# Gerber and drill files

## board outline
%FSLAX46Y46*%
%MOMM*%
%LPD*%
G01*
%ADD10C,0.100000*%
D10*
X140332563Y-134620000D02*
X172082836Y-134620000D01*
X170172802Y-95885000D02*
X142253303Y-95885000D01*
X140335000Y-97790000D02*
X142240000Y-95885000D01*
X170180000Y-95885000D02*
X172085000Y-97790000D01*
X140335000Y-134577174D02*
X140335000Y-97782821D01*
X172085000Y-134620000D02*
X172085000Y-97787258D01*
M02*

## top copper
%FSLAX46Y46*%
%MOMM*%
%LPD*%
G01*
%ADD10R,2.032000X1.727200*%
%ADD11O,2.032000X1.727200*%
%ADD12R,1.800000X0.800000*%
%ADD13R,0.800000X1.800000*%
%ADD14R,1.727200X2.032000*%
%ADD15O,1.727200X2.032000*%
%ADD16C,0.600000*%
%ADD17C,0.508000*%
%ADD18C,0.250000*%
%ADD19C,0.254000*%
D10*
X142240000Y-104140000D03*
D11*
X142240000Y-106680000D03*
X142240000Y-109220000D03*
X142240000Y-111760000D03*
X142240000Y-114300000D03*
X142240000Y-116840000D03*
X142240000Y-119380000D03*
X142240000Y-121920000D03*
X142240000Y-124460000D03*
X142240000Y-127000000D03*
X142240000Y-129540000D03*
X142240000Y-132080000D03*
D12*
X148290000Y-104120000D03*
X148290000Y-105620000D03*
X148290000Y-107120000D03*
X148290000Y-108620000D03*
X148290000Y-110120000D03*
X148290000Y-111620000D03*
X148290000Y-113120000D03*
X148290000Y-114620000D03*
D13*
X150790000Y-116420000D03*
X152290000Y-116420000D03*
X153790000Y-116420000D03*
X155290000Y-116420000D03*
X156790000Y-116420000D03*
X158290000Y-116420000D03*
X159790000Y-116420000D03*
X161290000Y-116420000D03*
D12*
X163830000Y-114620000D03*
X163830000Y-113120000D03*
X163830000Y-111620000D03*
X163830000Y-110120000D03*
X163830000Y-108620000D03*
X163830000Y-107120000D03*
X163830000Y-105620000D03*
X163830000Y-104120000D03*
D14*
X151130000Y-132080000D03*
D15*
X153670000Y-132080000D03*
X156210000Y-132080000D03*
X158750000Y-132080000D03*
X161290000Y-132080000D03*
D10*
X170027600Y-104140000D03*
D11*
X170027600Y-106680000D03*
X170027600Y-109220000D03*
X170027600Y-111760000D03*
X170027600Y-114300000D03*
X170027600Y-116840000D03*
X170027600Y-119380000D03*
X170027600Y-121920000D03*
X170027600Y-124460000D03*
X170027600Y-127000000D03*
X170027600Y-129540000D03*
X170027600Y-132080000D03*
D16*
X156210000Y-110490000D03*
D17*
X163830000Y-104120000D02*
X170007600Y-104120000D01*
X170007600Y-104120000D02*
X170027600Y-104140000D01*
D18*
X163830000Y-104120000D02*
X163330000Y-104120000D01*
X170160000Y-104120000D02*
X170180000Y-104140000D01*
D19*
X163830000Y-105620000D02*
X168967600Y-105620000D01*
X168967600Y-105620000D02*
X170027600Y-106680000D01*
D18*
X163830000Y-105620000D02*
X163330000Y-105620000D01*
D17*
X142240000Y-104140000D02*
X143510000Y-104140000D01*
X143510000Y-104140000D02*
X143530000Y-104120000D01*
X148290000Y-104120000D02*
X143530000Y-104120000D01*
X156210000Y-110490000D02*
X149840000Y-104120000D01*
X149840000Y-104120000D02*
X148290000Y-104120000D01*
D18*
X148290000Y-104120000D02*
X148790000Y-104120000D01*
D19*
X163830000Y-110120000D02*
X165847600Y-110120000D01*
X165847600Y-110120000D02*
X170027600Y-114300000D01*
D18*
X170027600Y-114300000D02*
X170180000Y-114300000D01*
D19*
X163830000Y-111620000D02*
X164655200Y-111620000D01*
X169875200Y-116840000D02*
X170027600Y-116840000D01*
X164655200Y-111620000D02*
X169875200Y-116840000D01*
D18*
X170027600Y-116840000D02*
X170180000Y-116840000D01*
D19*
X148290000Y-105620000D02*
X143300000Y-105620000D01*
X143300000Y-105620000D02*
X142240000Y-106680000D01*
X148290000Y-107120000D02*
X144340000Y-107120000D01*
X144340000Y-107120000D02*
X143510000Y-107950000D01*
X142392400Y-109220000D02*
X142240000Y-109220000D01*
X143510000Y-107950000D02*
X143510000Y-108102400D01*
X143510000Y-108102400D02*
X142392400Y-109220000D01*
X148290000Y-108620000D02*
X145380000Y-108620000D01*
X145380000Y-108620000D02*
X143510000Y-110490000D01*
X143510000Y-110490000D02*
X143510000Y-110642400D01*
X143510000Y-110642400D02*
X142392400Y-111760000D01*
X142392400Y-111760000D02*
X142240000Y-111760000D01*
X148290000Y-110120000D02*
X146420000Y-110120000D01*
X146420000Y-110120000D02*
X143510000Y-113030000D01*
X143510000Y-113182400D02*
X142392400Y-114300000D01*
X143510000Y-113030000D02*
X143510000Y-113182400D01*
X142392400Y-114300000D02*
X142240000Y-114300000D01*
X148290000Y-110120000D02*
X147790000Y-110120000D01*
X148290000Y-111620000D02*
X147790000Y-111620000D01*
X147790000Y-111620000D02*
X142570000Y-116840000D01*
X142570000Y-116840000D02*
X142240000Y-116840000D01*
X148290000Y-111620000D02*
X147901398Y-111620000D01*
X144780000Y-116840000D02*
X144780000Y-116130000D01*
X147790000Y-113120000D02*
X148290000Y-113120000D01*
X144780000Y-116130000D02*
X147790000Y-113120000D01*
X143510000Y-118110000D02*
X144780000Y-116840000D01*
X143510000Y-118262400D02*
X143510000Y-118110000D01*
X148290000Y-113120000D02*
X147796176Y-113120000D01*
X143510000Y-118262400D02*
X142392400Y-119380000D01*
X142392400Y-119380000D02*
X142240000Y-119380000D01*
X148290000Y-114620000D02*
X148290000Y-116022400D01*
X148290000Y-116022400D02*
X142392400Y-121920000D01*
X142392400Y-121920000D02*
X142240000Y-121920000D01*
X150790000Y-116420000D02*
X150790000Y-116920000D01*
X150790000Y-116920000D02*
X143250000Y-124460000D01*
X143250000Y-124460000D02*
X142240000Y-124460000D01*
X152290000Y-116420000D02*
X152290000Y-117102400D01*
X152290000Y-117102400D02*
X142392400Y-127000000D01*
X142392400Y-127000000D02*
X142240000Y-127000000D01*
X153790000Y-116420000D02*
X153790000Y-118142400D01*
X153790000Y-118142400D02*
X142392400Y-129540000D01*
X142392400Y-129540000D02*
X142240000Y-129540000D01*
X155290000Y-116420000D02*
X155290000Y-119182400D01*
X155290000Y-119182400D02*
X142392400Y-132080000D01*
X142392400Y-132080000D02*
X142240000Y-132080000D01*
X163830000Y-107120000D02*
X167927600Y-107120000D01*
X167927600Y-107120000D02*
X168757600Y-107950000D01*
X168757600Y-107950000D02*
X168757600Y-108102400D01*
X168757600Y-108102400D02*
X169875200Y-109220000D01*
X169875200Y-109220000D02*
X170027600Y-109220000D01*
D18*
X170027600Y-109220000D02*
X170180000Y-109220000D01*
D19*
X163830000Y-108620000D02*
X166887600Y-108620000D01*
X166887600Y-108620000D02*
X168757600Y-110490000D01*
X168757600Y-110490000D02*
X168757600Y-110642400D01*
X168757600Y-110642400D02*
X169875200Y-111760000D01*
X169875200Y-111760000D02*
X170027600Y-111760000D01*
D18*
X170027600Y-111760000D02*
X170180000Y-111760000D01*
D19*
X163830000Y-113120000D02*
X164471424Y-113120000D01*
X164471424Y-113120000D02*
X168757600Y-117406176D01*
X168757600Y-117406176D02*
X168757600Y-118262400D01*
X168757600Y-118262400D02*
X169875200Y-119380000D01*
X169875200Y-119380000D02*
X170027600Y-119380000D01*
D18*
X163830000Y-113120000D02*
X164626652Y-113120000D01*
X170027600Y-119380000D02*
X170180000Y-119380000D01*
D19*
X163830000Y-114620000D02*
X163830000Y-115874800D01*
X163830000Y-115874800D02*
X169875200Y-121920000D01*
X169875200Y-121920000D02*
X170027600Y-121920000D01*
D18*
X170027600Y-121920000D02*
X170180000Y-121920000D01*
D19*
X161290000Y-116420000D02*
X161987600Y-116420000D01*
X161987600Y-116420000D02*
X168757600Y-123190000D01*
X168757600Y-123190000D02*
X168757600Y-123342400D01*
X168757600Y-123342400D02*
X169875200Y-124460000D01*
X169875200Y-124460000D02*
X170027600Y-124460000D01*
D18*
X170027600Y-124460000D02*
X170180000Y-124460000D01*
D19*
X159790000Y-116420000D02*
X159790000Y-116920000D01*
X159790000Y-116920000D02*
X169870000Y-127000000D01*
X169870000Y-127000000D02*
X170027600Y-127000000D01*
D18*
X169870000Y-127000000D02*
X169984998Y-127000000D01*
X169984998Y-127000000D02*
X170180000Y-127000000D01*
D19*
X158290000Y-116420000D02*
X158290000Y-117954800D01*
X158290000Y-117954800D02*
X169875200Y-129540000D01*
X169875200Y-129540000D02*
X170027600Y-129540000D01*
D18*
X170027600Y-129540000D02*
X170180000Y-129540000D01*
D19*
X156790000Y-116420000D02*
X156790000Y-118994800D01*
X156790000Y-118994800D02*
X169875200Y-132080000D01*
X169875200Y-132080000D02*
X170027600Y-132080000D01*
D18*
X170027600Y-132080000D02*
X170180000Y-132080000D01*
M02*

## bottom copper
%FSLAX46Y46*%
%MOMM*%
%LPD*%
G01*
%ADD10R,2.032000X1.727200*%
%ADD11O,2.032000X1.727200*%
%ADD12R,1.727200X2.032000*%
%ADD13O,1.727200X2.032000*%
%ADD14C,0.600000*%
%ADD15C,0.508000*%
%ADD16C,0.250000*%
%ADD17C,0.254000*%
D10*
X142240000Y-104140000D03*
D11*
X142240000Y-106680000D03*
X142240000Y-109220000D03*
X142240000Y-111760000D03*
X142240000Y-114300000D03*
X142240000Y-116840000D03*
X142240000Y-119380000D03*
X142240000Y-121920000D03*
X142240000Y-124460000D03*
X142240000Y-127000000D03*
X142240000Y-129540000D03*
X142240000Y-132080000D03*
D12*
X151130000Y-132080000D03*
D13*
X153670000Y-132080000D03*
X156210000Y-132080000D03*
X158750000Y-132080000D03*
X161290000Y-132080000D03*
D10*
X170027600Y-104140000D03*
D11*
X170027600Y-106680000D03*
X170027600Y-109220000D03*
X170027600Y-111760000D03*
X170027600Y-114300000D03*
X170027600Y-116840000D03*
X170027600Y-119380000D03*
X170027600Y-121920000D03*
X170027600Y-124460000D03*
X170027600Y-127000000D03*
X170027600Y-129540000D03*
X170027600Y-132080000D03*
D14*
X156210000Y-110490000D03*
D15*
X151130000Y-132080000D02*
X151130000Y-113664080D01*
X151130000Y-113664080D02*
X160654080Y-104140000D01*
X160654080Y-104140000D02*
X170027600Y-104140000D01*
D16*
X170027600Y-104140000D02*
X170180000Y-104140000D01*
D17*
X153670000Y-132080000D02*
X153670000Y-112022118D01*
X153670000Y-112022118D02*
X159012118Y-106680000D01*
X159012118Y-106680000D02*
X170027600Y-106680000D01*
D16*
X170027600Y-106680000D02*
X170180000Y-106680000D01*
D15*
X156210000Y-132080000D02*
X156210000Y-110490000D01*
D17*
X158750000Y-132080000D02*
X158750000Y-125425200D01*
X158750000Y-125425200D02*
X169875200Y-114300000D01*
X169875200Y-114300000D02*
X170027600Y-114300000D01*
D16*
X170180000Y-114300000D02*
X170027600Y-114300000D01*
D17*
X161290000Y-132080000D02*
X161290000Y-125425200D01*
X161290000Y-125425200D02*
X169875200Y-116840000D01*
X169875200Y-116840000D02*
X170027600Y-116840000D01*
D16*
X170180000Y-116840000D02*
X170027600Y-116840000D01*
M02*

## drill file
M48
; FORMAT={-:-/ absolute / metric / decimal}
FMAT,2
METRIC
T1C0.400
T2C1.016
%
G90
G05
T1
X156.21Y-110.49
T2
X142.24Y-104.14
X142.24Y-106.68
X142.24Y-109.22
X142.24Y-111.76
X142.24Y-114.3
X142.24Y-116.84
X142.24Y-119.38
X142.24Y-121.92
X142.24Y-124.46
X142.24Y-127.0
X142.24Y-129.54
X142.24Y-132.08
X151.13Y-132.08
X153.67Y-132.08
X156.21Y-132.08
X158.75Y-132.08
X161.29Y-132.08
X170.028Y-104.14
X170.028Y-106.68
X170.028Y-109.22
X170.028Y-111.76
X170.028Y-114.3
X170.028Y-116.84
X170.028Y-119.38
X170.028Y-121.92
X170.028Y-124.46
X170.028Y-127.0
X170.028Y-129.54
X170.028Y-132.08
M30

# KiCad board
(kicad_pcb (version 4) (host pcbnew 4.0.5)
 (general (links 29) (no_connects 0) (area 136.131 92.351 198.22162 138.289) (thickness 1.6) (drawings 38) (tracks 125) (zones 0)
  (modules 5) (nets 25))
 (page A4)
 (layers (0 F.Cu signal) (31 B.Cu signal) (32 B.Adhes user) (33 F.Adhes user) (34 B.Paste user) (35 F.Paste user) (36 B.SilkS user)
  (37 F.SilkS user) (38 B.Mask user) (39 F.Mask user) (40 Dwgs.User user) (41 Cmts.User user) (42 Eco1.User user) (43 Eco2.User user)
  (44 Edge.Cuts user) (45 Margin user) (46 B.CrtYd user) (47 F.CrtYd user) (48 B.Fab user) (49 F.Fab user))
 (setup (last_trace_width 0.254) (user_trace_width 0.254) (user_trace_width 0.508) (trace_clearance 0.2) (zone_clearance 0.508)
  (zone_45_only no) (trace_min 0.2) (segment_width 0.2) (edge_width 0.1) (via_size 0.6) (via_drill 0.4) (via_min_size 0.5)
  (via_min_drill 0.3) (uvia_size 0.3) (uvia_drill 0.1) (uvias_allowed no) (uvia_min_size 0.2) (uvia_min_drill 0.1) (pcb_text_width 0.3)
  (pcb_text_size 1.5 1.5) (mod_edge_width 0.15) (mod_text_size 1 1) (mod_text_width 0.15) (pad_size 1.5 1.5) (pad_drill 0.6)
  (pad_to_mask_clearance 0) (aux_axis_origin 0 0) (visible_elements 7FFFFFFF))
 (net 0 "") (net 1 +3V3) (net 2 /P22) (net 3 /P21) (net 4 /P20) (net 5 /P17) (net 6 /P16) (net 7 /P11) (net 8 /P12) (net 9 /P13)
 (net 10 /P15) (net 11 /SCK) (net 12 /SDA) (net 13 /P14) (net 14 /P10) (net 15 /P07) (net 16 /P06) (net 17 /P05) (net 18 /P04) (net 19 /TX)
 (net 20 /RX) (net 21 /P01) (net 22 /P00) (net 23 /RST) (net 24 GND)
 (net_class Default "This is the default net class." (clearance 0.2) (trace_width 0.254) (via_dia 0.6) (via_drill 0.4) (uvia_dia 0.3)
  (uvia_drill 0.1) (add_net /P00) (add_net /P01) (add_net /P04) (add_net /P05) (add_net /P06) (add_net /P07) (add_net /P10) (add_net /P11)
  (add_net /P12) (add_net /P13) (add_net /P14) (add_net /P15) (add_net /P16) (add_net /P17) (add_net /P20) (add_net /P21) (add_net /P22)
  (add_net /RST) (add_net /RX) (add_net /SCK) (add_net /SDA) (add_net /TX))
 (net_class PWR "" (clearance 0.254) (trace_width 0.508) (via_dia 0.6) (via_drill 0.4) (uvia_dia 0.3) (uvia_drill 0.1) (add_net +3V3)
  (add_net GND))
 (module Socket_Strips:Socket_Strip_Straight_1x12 (layer F.Cu) (at 142.24 104.14 270)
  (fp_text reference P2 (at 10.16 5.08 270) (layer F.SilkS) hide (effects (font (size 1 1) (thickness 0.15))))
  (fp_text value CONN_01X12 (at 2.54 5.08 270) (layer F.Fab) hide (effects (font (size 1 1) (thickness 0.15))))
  (pad 1 thru_hole rect (at 0 0 270) (size 1.7272 2.032) (drill 1.016) (layers *.Cu *.Mask) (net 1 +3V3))
  (pad 2 thru_hole oval (at 2.54 0 270) (size 1.7272 2.032) (drill 1.016) (layers *.Cu *.Mask) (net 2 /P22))
  (pad 3 thru_hole oval (at 5.08 0 270) (size 1.7272 2.032) (drill 1.016) (layers *.Cu *.Mask) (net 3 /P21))
  (pad 4 thru_hole oval (at 7.62 0 270) (size 1.7272 2.032) (drill 1.016) (layers *.Cu *.Mask) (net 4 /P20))
  (pad 5 thru_hole oval (at 10.16 0 270) (size 1.7272 2.032) (drill 1.016) (layers *.Cu *.Mask) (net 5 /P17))
  (pad 6 thru_hole oval (at 12.7 0 270) (size 1.7272 2.032) (drill 1.016) (layers *.Cu *.Mask) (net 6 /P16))
  (pad 7 thru_hole oval (at 15.24 0 270) (size 1.7272 2.032) (drill 1.016) (layers *.Cu *.Mask) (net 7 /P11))
  (pad 8 thru_hole oval (at 17.78 0 270) (size 1.7272 2.032) (drill 1.016) (layers *.Cu *.Mask) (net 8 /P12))
  (pad 9 thru_hole oval (at 20.32 0 270) (size 1.7272 2.032) (drill 1.016) (layers *.Cu *.Mask) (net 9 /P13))
  (pad 10 thru_hole oval (at 22.86 0 270) (size 1.7272 2.032) (drill 1.016) (layers *.Cu *.Mask) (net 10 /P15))
  (pad 11 thru_hole oval (at 25.4 0 270) (size 1.7272 2.032) (drill 1.016) (layers *.Cu *.Mask) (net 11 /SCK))
  (pad 12 thru_hole oval (at 27.94 0 270) (size 1.7272 2.032) (drill 1.016) (layers *.Cu *.Mask) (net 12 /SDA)))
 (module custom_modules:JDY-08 (layer F.Cu) (at 148.59 96.52)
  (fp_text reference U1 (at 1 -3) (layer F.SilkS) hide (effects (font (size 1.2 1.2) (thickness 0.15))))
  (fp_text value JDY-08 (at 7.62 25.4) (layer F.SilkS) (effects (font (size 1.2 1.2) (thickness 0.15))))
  (pad 1 smd rect (at -0.3 7.6 90) (size 0.8 1.8) (layers F.Cu F.Paste F.Mask) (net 1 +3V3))
  (pad 2 smd rect (at -0.3 9.1 90) (size 0.8 1.8) (layers F.Cu F.Paste F.Mask) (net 2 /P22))
  (pad 3 smd rect (at -0.3 10.6 90) (size 0.8 1.8) (layers F.Cu F.Paste F.Mask) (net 3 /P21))
  (pad 4 smd rect (at -0.3 12.1 90) (size 0.8 1.8) (layers F.Cu F.Paste F.Mask) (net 4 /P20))
  (pad 5 smd rect (at -0.3 13.6 90) (size 0.8 1.8) (layers F.Cu F.Paste F.Mask) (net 5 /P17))
  (pad 6 smd rect (at -0.3 15.1 90) (size 0.8 1.8) (layers F.Cu F.Paste F.Mask) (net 6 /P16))
  (pad 7 smd rect (at -0.3 16.6 90) (size 0.8 1.8) (layers F.Cu F.Paste F.Mask) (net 7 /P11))
  (pad 8 smd rect (at -0.3 18.1 90) (size 0.8 1.8) (layers F.Cu F.Paste F.Mask) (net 8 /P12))
  (pad 9 smd rect (at 2.2 19.9) (size 0.8 1.8) (layers F.Cu F.Paste F.Mask) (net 9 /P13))
  (pad 10 smd rect (at 3.7 19.9) (size 0.8 1.8) (layers F.Cu F.Paste F.Mask) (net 10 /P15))
  (pad 11 smd rect (at 5.2 19.9) (size 0.8 1.8) (layers F.Cu F.Paste F.Mask) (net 11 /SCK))
  (pad 12 smd rect (at 6.7 19.9) (size 0.8 1.8) (layers F.Cu F.Paste F.Mask) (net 12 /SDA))
  (pad 13 smd rect (at 8.2 19.9) (size 0.8 1.8) (layers F.Cu F.Paste F.Mask) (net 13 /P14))
  (pad 14 smd rect (at 9.7 19.9) (size 0.8 1.8) (layers F.Cu F.Paste F.Mask) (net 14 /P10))
  (pad 15 smd rect (at 11.2 19.9) (size 0.8 1.8) (layers F.Cu F.Paste F.Mask) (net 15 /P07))
  (pad 16 smd rect (at 12.7 19.9) (size 0.8 1.8) (layers F.Cu F.Paste F.Mask) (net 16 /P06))
  (pad 17 smd rect (at 15.24 18.1 90) (size 0.8 1.8) (layers F.Cu F.Paste F.Mask) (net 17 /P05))
  (pad 18 smd rect (at 15.24 16.6 90) (size 0.8 1.8) (layers F.Cu F.Paste F.Mask) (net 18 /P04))
  (pad 19 smd rect (at 15.24 15.1 90) (size 0.8 1.8) (layers F.Cu F.Paste F.Mask) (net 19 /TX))
  (pad 20 smd rect (at 15.24 13.6 90) (size 0.8 1.8) (layers F.Cu F.Paste F.Mask) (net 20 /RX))
  (pad 21 smd rect (at 15.24 12.1 90) (size 0.8 1.8) (layers F.Cu F.Paste F.Mask) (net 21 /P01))
  (pad 22 smd rect (at 15.24 10.6 90) (size 0.8 1.8) (layers F.Cu F.Paste F.Mask) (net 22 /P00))
  (pad 23 smd rect (at 15.24 9.1 90) (size 0.8 1.8) (layers F.Cu F.Paste F.Mask) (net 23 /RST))
  (pad 24 smd rect (at 15.24 7.6 90) (size 0.8 1.8) (layers F.Cu F.Paste F.Mask) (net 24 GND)))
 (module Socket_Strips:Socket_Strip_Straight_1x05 (layer F.Cu) (at 151.13 132.08)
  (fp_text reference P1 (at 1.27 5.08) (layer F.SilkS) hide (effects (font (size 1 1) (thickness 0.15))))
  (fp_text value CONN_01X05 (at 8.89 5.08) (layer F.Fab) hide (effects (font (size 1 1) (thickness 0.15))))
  (pad 1 thru_hole rect (at 0 0) (size 1.7272 2.032) (drill 1.016) (layers *.Cu *.Mask) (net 24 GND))
  (pad 2 thru_hole oval (at 2.54 0) (size 1.7272 2.032) (drill 1.016) (layers *.Cu *.Mask) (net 23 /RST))
  (pad 3 thru_hole oval (at 5.08 0) (size 1.7272 2.032) (drill 1.016) (layers *.Cu *.Mask) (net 1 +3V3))
  (pad 4 thru_hole oval (at 7.62 0) (size 1.7272 2.032) (drill 1.016) (layers *.Cu *.Mask) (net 20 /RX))
  (pad 5 thru_hole oval (at 10.16 0) (size 1.7272 2.032) (drill 1.016) (layers *.Cu *.Mask) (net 19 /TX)))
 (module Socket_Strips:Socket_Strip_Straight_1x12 (layer F.Cu) (at 170.0276 104.14 270)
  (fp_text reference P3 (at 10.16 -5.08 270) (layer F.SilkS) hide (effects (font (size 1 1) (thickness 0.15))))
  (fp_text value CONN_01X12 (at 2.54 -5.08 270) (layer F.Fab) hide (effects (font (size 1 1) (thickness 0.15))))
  (pad 1 thru_hole rect (at 0 0 270) (size 1.7272 2.032) (drill 1.016) (layers *.Cu *.Mask) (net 24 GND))
  (pad 2 thru_hole oval (at 2.54 0 270) (size 1.7272 2.032) (drill 1.016) (layers *.Cu *.Mask) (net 23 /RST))
  (pad 3 thru_hole oval (at 5.08 0 270) (size 1.7272 2.032) (drill 1.016) (layers *.Cu *.Mask) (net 22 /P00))
  (pad 4 thru_hole oval (at 7.62 0 270) (size 1.7272 2.032) (drill 1.016) (layers *.Cu *.Mask) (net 21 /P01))
  (pad 5 thru_hole oval (at 10.16 0 270) (size 1.7272 2.032) (drill 1.016) (layers *.Cu *.Mask) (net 20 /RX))
  (pad 6 thru_hole oval (at 12.7 0 270) (size 1.7272 2.032) (drill 1.016) (layers *.Cu *.Mask) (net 19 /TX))
  (pad 7 thru_hole oval (at 15.24 0 270) (size 1.7272 2.032) (drill 1.016) (layers *.Cu *.Mask) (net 18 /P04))
  (pad 8 thru_hole oval (at 17.78 0 270) (size 1.7272 2.032) (drill 1.016) (layers *.Cu *.Mask) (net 17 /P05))
  (pad 9 thru_hole oval (at 20.32 0 270) (size 1.7272 2.032) (drill 1.016) (layers *.Cu *.Mask) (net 16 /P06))
  (pad 10 thru_hole oval (at 22.86 0 270) (size 1.7272 2.032) (drill 1.016) (layers *.Cu *.Mask) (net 15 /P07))
  (pad 11 thru_hole oval (at 25.4 0 270) (size 1.7272 2.032) (drill 1.016) (layers *.Cu *.Mask) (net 14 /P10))
  (pad 12 thru_hole oval (at 27.94 0 270) (size 1.7272 2.032) (drill 1.016) (layers *.Cu *.Mask) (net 13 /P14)))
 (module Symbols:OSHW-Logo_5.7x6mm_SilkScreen (layer F.Cu) (at 149.86 124.46)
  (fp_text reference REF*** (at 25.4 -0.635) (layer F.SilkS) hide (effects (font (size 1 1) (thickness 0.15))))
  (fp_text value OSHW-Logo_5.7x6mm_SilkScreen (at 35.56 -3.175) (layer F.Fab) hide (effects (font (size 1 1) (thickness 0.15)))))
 (gr_line (start 140.332563 134.62) (end 172.082836 134.62) (layer Edge.Cuts) (width 0.1))
 (gr_line (start 170.172802 95.885) (end 142.253303 95.885) (layer Edge.Cuts) (width 0.1))
 (gr_line (start 140.335 97.79) (end 142.24 95.885) (layer Edge.Cuts) (width 0.1))
 (gr_line (start 170.18 95.885) (end 172.085 97.79) (layer Edge.Cuts) (width 0.1))
 (gr_line (start 140.335 134.577174) (end 140.335 97.782821) (layer Edge.Cuts) (width 0.1))
 (gr_line (start 172.085 134.62) (end 172.085 97.787258) (layer Edge.Cuts) (width 0.1))
 (segment (start 151.13 132.08) (end 151.13 113.66408) (width 0.508) (layer B.Cu) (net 24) (status 10))
 (segment (start 151.13 113.66408) (end 160.65408 104.14) (width 0.508) (layer B.Cu) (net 24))
 (segment (start 160.65408 104.14) (end 170.0276 104.14) (width 0.508) (layer B.Cu) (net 24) (status 20))
 (segment (start 163.83 104.12) (end 170.0076 104.12) (width 0.508) (layer F.Cu) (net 24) (status 30))
 (segment (start 170.0076 104.12) (end 170.0276 104.14) (width 0.508) (layer F.Cu) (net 24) (status 30))
 (segment (start 170.0276 104.14) (end 170.18 104.14) (width 0.25) (layer B.Cu) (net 24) (status 30))
 (segment (start 163.83 104.12) (end 163.33 104.12) (width 0.25) (layer F.Cu) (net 24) (status 30))
 (segment (start 170.16 104.12) (end 170.18 104.14) (width 0.25) (layer F.Cu) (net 24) (status 30))
 (segment (start 153.67 132.08) (end 153.67 112.022118) (width 0.254) (layer B.Cu) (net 23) (status 10))
 (segment (start 153.67 112.022118) (end 159.012118 106.68) (width 0.254) (layer B.Cu) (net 23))
 (segment (start 159.012118 106.68) (end 170.0276 106.68) (width 0.254) (layer B.Cu) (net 23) (status 20))
 (segment (start 163.83 105.62) (end 168.9676 105.62) (width 0.254) (layer F.Cu) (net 23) (status 10))
 (segment (start 168.9676 105.62) (end 170.0276 106.68) (width 0.254) (layer F.Cu) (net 23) (status 20))
 (segment (start 170.0276 106.68) (end 170.18 106.68) (width 0.25) (layer B.Cu) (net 23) (status 30))
 (segment (start 163.83 105.62) (end 163.33 105.62) (width 0.25) (layer F.Cu) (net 23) (status 30))
 (segment (start 142.24 104.14) (end 143.51 104.14) (width 0.508) (layer F.Cu) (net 1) (status 10))
 (segment (start 143.51 104.14) (end 143.53 104.12) (width 0.508) (layer F.Cu) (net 1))
 (segment (start 148.29 104.12) (end 143.53 104.12) (width 0.508) (layer F.Cu) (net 1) (status 10))
 (segment (start 156.21 110.49) (end 149.84 104.12) (width 0.508) (layer F.Cu) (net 1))
 (segment (start 149.84 104.12) (end 148.29 104.12) (width 0.508) (layer F.Cu) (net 1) (status 20))
 (segment (start 156.21 132.08) (end 156.21 110.49) (width 0.508) (layer B.Cu) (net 1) (status 10))
 (segment (start 148.29 104.12) (end 148.79 104.12) (width 0.25) (layer F.Cu) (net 1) (status 30))
 (segment (start 158.75 132.08) (end 158.75 125.4252) (width 0.254) (layer B.Cu) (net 20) (status 10))
 (segment (start 158.75 125.4252) (end 169.8752 114.3) (width 0.254) (layer B.Cu) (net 20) (status 20))
 (segment (start 169.8752 114.3) (end 170.0276 114.3) (width 0.254) (layer B.Cu) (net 20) (status 30))
 (segment (start 163.83 110.12) (end 165.8476 110.12) (width 0.254) (layer F.Cu) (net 20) (status 10))
 (segment (start 165.8476 110.12) (end 170.0276 114.3) (width 0.254) (layer F.Cu) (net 20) (status 20))
 (segment (start 170.18 114.3) (end 170.0276 114.3) (width 0.25) (layer B.Cu) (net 20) (status 30))
 (segment (start 170.0276 114.3) (end 170.18 114.3) (width 0.25) (layer F.Cu) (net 20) (status 30))
 (segment (start 161.29 132.08) (end 161.29 125.4252) (width 0.254) (layer B.Cu) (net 19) (status 10))
 (segment (start 161.29 125.4252) (end 169.8752 116.84) (width 0.254) (layer B.Cu) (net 19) (status 20))
 (segment (start 169.8752 116.84) (end 170.0276 116.84) (width 0.254) (layer B.Cu) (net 19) (status 30))
 (segment (start 163.83 111.62) (end 164.6552 111.62) (width 0.254) (layer F.Cu) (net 19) (status 30))
 (segment (start 169.8752 116.84) (end 170.0276 116.84) (width 0.254) (layer F.Cu) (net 19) (status 30))
 (segment (start 164.6552 111.62) (end 169.8752 116.84) (width 0.254) (layer F.Cu) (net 19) (status 30))
 (segment (start 170.18 116.84) (end 170.0276 116.84) (width 0.25) (layer B.Cu) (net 19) (status 30))
 (segment (start 170.0276 116.84) (end 170.18 116.84) (width 0.25) (layer F.Cu) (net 19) (status 30))
 (segment (start 148.29 105.62) (end 143.3 105.62) (width 0.254) (layer F.Cu) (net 2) (status 10))
 (segment (start 143.3 105.62) (end 142.24 106.68) (width 0.254) (layer F.Cu) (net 2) (status 20))
 (segment (start 148.29 107.12) (end 144.34 107.12) (width 0.254) (layer F.Cu) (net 3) (status 10))
 (segment (start 144.34 107.12) (end 143.51 107.95) (width 0.254) (layer F.Cu) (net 3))
 (segment (start 142.3924 109.22) (end 142.24 109.22) (width 0.254) (layer F.Cu) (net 3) (status 30))
 (segment (start 143.51 107.95) (end 143.51 108.1024) (width 0.254) (layer F.Cu) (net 3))
 (segment (start 143.51 108.1024) (end 142.3924 109.22) (width 0.254) (layer F.Cu) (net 3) (status 20))
 (segment (start 148.29 108.62) (end 145.38 108.62) (width 0.254) (layer F.Cu) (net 4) (status 10))
 (segment (start 145.38 108.62) (end 143.51 110.49) (width 0.254) (layer F.Cu) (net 4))
 (segment (start 143.51 110.49) (end 143.51 110.6424) (width 0.254) (layer F.Cu) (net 4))
 (segment (start 143.51 110.6424) (end 142.3924 111.76) (width 0.254) (layer F.Cu) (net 4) (status 20))
 (segment (start 142.3924 111.76) (end 142.24 111.76) (width 0.254) (layer F.Cu) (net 4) (status 30))
 (segment (start 148.29 110.12) (end 146.42 110.12) (width 0.254) (layer F.Cu) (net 5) (status 10))
 (segment (start 146.42 110.12) (end 143.51 113.03) (width 0.254) (layer F.Cu) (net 5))
 (segment (start 143.51 113.1824) (end 142.3924 114.3) (width 0.254) (layer F.Cu) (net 5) (status 20))
 (segment (start 143.51 113.03) (end 143.51 113.1824) (width 0.254) (layer F.Cu) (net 5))
 (segment (start 142.3924 114.3) (end 142.24 114.3) (width 0.254) (layer F.Cu) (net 5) (status 30))
 (segment (start 148.29 110.12) (end 147.79 110.12) (width 0.254) (layer F.Cu) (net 5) (status 30))
 (segment (start 148.29 111.62) (end 147.79 111.62) (width 0.254) (layer F.Cu) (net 6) (status 30))
 (segment (start 147.79 111.62) (end 142.57 116.84) (width 0.254) (layer F.Cu) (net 6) (status 30))
 (segment (start 142.57 116.84) (end 142.24 116.84) (width 0.254) (layer F.Cu) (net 6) (status 30))
 (segment (start 148.29 111.62) (end 147.901398 111.62) (width 0.254) (layer F.Cu) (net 6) (status 30))
 (segment (start 144.78 116.84) (end 144.78 116.13) (width 0.254) (layer F.Cu) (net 7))
 (segment (start 147.79 113.12) (end 148.29 113.12) (width 0.254) (layer F.Cu) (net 7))
 (segment (start 144.78 116.13) (end 147.79 113.12) (width 0.254) (layer F.Cu) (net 7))
 (segment (start 143.51 118.11) (end 144.78 116.84) (width 0.254) (layer F.Cu) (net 7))
 (segment (start 143.51 118.2624) (end 143.51 118.11) (width 0.254) (layer F.Cu) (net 7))
 (segment (start 148.29 113.12) (end 147.796176 113.12) (width 0.254) (layer F.Cu) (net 7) (status 30))
 (segment (start 143.51 118.2624) (end 142.3924 119.38) (width 0.254) (layer F.Cu) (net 7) (status 20))
 (segment (start 142.3924 119.38) (end 142.24 119.38) (width 0.254) (layer F.Cu) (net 7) (status 30))
 (segment (start 148.29 114.62) (end 148.29 116.0224) (width 0.254) (layer F.Cu) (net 8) (status 10))
 (segment (start 148.29 116.0224) (end 142.3924 121.92) (width 0.254) (layer F.Cu) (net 8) (status 20))
 (segment (start 142.3924 121.92) (end 142.24 121.92) (width 0.254) (layer F.Cu) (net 8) (status 30))
 (segment (start 150.79 116.42) (end 150.79 116.92) (width 0.254) (layer F.Cu) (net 9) (status 30))
 (segment (start 150.79 116.92) (end 143.25 124.46) (width 0.254) (layer F.Cu) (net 9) (status 30))
 (segment (start 143.25 124.46) (end 142.24 124.46) (width 0.254) (layer F.Cu) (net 9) (status 30))
 (segment (start 152.29 116.42) (end 152.29 117.1024) (width 0.254) (layer F.Cu) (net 10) (status 30))
 (segment (start 152.29 117.1024) (end 142.3924 127) (width 0.254) (layer F.Cu) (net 10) (status 30))
 (segment (start 142.3924 127) (end 142.24 127) (width 0.254) (layer F.Cu) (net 10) (status 30))
 (segment (start 153.79 116.42) (end 153.79 118.1424) (width 0.254) (layer F.Cu) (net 11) (status 10))
 (segment (start 153.79 118.1424) (end 142.3924 129.54) (width 0.254) (layer F.Cu) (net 11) (status 20))
 (segment (start 142.3924 129.54) (end 142.24 129.54) (width 0.254) (layer F.Cu) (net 11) (status 30))
 (segment (start 155.29 116.42) (end 155.29 119.1824) (width 0.254) (layer F.Cu) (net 12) (status 10))
 (segment (start 155.29 119.1824) (end 142.3924 132.08) (width 0.254) (layer F.Cu) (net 12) (status 20))
 (segment (start 142.3924 132.08) (end 142.24 132.08) (width 0.254) (layer F.Cu) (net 12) (status 30))
 (segment (start 163.83 107.12) (end 167.9276 107.12) (width 0.254) (layer F.Cu) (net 22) (status 10))
 (segment (start 167.9276 107.12) (end 168.7576 107.95) (width 0.254) (layer F.Cu) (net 22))
 (segment (start 168.7576 107.95) (end 168.7576 108.1024) (width 0.254) (layer F.Cu) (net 22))
 (segment (start 168.7576 108.1024) (end 169.8752 109.22) (width 0.254) (layer F.Cu) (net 22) (status 20))
 (segment (start 169.8752 109.22) (end 170.0276 109.22) (width 0.254) (layer F.Cu) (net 22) (status 30))
 (segment (start 170.0276 109.22) (end 170.18 109.22) (width 0.25) (layer F.Cu) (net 22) (status 30))
 (segment (start 163.83 108.62) (end 166.8876 108.62) (width 0.254) (layer F.Cu) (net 21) (status 10))
 (segment (start 166.8876 108.62) (end 168.7576 110.49) (width 0.254) (layer F.Cu) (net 21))
 (segment (start 168.7576 110.49) (end 168.7576 110.6424) (width 0.254) (layer F.Cu) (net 21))
 (segment (start 168.7576 110.6424) (end 169.8752 111.76) (width 0.254) (layer F.Cu) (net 21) (status 20))
 (segment (start 169.8752 111.76) (end 170.0276 111.76) (width 0.254) (layer F.Cu) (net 21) (status 30))
 (segment (start 170.0276 111.76) (end 170.18 111.76) (width 0.25) (layer F.Cu) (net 21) (status 30))
 (segment (start 163.83 113.12) (end 164.471424 113.12) (width 0.254) (layer F.Cu) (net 18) (status 30))
 (segment (start 164.471424 113.12) (end 168.7576 117.406176) (width 0.254) (layer F.Cu) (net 18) (status 10))
 (segment (start 168.7576 117.406176) (end 168.7576 118.2624) (width 0.254) (layer F.Cu) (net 18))
 (segment (start 168.7576 118.2624) (end 169.8752 119.38) (width 0.254) (layer F.Cu) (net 18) (status 20))
 (segment (start 169.8752 119.38) (end 170.0276 119.38) (width 0.254) (layer F.Cu) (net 18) (status 30))
 (segment (start 163.83 113.12) (end 164.626652 113.12) (width 0.25) (layer F.Cu) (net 18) (status 30))
 (segment (start 170.0276 119.38) (end 170.18 119.38) (width 0.25) (layer F.Cu) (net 18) (status 30))
 (segment (start 163.83 114.62) (end 163.83 115.8748) (width 0.254) (layer F.Cu) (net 17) (status 10))
 (segment (start 163.83 115.8748) (end 169.8752 121.92) (width 0.254) (layer F.Cu) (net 17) (status 20))
 (segment (start 169.8752 121.92) (end 170.0276 121.92) (width 0.254) (layer F.Cu) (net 17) (status 30))
 (segment (start 170.0276 121.92) (end 170.18 121.92) (width 0.25) (layer F.Cu) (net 17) (status 30))
 (segment (start 161.29 116.42) (end 161.9876 116.42) (width 0.254) (layer F.Cu) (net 16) (status 10))
 (segment (start 161.9876 116.42) (end 168.7576 123.19) (width 0.254) (layer F.Cu) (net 16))
 (segment (start 168.7576 123.19) (end 168.7576 123.3424) (width 0.254) (layer F.Cu) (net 16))
 (segment (start 168.7576 123.3424) (end 169.8752 124.46) (width 0.254) (layer F.Cu) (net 16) (status 20))
 (segment (start 169.8752 124.46) (end 170.0276 124.46) (width 0.254) (layer F.Cu) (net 16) (status 30))
 (segment (start 170.0276 124.46) (end 170.18 124.46) (width 0.25) (layer F.Cu) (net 16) (status 30))
 (segment (start 159.79 116.42) (end 159.79 116.92) (width 0.254) (layer F.Cu) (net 15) (status 30))
 (segment (start 159.79 116.92) (end 169.87 127) (width 0.254) (layer F.Cu) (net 15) (status 30))
 (segment (start 169.87 127) (end 170.0276 127) (width 0.254) (layer F.Cu) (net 15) (status 30))
 (segment (start 169.87 127) (end 169.984998 127) (width 0.25) (layer F.Cu) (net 15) (status 30))
 (segment (start 169.984998 127) (end 170.18 127) (width 0.25) (layer F.Cu) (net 15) (status 30))
 (segment (start 158.29 116.42) (end 158.29 117.9548) (width 0.254) (layer F.Cu) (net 14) (status 10))
 (segment (start 158.29 117.9548) (end 169.8752 129.54) (width 0.254) (layer F.Cu) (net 14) (status 20))
 (segment (start 169.8752 129.54) (end 170.0276 129.54) (width 0.254) (layer F.Cu) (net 14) (status 30))
 (segment (start 170.0276 129.54) (end 170.18 129.54) (width 0.25) (layer F.Cu) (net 14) (status 30))
 (segment (start 156.79 116.42) (end 156.79 118.9948) (width 0.254) (layer F.Cu) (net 13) (status 10))
 (segment (start 156.79 118.9948) (end 169.8752 132.08) (width 0.254) (layer F.Cu) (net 13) (status 20))
 (segment (start 169.8752 132.08) (end 170.0276 132.08) (width 0.254) (layer F.Cu) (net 13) (status 30))
 (segment (start 170.0276 132.08) (end 170.18 132.08) (width 0.25) (layer F.Cu) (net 13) (status 30))
 (via (at 156.21 110.49) (size 0.6) (drill 0.4) (layers F.Cu B.Cu) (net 1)))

